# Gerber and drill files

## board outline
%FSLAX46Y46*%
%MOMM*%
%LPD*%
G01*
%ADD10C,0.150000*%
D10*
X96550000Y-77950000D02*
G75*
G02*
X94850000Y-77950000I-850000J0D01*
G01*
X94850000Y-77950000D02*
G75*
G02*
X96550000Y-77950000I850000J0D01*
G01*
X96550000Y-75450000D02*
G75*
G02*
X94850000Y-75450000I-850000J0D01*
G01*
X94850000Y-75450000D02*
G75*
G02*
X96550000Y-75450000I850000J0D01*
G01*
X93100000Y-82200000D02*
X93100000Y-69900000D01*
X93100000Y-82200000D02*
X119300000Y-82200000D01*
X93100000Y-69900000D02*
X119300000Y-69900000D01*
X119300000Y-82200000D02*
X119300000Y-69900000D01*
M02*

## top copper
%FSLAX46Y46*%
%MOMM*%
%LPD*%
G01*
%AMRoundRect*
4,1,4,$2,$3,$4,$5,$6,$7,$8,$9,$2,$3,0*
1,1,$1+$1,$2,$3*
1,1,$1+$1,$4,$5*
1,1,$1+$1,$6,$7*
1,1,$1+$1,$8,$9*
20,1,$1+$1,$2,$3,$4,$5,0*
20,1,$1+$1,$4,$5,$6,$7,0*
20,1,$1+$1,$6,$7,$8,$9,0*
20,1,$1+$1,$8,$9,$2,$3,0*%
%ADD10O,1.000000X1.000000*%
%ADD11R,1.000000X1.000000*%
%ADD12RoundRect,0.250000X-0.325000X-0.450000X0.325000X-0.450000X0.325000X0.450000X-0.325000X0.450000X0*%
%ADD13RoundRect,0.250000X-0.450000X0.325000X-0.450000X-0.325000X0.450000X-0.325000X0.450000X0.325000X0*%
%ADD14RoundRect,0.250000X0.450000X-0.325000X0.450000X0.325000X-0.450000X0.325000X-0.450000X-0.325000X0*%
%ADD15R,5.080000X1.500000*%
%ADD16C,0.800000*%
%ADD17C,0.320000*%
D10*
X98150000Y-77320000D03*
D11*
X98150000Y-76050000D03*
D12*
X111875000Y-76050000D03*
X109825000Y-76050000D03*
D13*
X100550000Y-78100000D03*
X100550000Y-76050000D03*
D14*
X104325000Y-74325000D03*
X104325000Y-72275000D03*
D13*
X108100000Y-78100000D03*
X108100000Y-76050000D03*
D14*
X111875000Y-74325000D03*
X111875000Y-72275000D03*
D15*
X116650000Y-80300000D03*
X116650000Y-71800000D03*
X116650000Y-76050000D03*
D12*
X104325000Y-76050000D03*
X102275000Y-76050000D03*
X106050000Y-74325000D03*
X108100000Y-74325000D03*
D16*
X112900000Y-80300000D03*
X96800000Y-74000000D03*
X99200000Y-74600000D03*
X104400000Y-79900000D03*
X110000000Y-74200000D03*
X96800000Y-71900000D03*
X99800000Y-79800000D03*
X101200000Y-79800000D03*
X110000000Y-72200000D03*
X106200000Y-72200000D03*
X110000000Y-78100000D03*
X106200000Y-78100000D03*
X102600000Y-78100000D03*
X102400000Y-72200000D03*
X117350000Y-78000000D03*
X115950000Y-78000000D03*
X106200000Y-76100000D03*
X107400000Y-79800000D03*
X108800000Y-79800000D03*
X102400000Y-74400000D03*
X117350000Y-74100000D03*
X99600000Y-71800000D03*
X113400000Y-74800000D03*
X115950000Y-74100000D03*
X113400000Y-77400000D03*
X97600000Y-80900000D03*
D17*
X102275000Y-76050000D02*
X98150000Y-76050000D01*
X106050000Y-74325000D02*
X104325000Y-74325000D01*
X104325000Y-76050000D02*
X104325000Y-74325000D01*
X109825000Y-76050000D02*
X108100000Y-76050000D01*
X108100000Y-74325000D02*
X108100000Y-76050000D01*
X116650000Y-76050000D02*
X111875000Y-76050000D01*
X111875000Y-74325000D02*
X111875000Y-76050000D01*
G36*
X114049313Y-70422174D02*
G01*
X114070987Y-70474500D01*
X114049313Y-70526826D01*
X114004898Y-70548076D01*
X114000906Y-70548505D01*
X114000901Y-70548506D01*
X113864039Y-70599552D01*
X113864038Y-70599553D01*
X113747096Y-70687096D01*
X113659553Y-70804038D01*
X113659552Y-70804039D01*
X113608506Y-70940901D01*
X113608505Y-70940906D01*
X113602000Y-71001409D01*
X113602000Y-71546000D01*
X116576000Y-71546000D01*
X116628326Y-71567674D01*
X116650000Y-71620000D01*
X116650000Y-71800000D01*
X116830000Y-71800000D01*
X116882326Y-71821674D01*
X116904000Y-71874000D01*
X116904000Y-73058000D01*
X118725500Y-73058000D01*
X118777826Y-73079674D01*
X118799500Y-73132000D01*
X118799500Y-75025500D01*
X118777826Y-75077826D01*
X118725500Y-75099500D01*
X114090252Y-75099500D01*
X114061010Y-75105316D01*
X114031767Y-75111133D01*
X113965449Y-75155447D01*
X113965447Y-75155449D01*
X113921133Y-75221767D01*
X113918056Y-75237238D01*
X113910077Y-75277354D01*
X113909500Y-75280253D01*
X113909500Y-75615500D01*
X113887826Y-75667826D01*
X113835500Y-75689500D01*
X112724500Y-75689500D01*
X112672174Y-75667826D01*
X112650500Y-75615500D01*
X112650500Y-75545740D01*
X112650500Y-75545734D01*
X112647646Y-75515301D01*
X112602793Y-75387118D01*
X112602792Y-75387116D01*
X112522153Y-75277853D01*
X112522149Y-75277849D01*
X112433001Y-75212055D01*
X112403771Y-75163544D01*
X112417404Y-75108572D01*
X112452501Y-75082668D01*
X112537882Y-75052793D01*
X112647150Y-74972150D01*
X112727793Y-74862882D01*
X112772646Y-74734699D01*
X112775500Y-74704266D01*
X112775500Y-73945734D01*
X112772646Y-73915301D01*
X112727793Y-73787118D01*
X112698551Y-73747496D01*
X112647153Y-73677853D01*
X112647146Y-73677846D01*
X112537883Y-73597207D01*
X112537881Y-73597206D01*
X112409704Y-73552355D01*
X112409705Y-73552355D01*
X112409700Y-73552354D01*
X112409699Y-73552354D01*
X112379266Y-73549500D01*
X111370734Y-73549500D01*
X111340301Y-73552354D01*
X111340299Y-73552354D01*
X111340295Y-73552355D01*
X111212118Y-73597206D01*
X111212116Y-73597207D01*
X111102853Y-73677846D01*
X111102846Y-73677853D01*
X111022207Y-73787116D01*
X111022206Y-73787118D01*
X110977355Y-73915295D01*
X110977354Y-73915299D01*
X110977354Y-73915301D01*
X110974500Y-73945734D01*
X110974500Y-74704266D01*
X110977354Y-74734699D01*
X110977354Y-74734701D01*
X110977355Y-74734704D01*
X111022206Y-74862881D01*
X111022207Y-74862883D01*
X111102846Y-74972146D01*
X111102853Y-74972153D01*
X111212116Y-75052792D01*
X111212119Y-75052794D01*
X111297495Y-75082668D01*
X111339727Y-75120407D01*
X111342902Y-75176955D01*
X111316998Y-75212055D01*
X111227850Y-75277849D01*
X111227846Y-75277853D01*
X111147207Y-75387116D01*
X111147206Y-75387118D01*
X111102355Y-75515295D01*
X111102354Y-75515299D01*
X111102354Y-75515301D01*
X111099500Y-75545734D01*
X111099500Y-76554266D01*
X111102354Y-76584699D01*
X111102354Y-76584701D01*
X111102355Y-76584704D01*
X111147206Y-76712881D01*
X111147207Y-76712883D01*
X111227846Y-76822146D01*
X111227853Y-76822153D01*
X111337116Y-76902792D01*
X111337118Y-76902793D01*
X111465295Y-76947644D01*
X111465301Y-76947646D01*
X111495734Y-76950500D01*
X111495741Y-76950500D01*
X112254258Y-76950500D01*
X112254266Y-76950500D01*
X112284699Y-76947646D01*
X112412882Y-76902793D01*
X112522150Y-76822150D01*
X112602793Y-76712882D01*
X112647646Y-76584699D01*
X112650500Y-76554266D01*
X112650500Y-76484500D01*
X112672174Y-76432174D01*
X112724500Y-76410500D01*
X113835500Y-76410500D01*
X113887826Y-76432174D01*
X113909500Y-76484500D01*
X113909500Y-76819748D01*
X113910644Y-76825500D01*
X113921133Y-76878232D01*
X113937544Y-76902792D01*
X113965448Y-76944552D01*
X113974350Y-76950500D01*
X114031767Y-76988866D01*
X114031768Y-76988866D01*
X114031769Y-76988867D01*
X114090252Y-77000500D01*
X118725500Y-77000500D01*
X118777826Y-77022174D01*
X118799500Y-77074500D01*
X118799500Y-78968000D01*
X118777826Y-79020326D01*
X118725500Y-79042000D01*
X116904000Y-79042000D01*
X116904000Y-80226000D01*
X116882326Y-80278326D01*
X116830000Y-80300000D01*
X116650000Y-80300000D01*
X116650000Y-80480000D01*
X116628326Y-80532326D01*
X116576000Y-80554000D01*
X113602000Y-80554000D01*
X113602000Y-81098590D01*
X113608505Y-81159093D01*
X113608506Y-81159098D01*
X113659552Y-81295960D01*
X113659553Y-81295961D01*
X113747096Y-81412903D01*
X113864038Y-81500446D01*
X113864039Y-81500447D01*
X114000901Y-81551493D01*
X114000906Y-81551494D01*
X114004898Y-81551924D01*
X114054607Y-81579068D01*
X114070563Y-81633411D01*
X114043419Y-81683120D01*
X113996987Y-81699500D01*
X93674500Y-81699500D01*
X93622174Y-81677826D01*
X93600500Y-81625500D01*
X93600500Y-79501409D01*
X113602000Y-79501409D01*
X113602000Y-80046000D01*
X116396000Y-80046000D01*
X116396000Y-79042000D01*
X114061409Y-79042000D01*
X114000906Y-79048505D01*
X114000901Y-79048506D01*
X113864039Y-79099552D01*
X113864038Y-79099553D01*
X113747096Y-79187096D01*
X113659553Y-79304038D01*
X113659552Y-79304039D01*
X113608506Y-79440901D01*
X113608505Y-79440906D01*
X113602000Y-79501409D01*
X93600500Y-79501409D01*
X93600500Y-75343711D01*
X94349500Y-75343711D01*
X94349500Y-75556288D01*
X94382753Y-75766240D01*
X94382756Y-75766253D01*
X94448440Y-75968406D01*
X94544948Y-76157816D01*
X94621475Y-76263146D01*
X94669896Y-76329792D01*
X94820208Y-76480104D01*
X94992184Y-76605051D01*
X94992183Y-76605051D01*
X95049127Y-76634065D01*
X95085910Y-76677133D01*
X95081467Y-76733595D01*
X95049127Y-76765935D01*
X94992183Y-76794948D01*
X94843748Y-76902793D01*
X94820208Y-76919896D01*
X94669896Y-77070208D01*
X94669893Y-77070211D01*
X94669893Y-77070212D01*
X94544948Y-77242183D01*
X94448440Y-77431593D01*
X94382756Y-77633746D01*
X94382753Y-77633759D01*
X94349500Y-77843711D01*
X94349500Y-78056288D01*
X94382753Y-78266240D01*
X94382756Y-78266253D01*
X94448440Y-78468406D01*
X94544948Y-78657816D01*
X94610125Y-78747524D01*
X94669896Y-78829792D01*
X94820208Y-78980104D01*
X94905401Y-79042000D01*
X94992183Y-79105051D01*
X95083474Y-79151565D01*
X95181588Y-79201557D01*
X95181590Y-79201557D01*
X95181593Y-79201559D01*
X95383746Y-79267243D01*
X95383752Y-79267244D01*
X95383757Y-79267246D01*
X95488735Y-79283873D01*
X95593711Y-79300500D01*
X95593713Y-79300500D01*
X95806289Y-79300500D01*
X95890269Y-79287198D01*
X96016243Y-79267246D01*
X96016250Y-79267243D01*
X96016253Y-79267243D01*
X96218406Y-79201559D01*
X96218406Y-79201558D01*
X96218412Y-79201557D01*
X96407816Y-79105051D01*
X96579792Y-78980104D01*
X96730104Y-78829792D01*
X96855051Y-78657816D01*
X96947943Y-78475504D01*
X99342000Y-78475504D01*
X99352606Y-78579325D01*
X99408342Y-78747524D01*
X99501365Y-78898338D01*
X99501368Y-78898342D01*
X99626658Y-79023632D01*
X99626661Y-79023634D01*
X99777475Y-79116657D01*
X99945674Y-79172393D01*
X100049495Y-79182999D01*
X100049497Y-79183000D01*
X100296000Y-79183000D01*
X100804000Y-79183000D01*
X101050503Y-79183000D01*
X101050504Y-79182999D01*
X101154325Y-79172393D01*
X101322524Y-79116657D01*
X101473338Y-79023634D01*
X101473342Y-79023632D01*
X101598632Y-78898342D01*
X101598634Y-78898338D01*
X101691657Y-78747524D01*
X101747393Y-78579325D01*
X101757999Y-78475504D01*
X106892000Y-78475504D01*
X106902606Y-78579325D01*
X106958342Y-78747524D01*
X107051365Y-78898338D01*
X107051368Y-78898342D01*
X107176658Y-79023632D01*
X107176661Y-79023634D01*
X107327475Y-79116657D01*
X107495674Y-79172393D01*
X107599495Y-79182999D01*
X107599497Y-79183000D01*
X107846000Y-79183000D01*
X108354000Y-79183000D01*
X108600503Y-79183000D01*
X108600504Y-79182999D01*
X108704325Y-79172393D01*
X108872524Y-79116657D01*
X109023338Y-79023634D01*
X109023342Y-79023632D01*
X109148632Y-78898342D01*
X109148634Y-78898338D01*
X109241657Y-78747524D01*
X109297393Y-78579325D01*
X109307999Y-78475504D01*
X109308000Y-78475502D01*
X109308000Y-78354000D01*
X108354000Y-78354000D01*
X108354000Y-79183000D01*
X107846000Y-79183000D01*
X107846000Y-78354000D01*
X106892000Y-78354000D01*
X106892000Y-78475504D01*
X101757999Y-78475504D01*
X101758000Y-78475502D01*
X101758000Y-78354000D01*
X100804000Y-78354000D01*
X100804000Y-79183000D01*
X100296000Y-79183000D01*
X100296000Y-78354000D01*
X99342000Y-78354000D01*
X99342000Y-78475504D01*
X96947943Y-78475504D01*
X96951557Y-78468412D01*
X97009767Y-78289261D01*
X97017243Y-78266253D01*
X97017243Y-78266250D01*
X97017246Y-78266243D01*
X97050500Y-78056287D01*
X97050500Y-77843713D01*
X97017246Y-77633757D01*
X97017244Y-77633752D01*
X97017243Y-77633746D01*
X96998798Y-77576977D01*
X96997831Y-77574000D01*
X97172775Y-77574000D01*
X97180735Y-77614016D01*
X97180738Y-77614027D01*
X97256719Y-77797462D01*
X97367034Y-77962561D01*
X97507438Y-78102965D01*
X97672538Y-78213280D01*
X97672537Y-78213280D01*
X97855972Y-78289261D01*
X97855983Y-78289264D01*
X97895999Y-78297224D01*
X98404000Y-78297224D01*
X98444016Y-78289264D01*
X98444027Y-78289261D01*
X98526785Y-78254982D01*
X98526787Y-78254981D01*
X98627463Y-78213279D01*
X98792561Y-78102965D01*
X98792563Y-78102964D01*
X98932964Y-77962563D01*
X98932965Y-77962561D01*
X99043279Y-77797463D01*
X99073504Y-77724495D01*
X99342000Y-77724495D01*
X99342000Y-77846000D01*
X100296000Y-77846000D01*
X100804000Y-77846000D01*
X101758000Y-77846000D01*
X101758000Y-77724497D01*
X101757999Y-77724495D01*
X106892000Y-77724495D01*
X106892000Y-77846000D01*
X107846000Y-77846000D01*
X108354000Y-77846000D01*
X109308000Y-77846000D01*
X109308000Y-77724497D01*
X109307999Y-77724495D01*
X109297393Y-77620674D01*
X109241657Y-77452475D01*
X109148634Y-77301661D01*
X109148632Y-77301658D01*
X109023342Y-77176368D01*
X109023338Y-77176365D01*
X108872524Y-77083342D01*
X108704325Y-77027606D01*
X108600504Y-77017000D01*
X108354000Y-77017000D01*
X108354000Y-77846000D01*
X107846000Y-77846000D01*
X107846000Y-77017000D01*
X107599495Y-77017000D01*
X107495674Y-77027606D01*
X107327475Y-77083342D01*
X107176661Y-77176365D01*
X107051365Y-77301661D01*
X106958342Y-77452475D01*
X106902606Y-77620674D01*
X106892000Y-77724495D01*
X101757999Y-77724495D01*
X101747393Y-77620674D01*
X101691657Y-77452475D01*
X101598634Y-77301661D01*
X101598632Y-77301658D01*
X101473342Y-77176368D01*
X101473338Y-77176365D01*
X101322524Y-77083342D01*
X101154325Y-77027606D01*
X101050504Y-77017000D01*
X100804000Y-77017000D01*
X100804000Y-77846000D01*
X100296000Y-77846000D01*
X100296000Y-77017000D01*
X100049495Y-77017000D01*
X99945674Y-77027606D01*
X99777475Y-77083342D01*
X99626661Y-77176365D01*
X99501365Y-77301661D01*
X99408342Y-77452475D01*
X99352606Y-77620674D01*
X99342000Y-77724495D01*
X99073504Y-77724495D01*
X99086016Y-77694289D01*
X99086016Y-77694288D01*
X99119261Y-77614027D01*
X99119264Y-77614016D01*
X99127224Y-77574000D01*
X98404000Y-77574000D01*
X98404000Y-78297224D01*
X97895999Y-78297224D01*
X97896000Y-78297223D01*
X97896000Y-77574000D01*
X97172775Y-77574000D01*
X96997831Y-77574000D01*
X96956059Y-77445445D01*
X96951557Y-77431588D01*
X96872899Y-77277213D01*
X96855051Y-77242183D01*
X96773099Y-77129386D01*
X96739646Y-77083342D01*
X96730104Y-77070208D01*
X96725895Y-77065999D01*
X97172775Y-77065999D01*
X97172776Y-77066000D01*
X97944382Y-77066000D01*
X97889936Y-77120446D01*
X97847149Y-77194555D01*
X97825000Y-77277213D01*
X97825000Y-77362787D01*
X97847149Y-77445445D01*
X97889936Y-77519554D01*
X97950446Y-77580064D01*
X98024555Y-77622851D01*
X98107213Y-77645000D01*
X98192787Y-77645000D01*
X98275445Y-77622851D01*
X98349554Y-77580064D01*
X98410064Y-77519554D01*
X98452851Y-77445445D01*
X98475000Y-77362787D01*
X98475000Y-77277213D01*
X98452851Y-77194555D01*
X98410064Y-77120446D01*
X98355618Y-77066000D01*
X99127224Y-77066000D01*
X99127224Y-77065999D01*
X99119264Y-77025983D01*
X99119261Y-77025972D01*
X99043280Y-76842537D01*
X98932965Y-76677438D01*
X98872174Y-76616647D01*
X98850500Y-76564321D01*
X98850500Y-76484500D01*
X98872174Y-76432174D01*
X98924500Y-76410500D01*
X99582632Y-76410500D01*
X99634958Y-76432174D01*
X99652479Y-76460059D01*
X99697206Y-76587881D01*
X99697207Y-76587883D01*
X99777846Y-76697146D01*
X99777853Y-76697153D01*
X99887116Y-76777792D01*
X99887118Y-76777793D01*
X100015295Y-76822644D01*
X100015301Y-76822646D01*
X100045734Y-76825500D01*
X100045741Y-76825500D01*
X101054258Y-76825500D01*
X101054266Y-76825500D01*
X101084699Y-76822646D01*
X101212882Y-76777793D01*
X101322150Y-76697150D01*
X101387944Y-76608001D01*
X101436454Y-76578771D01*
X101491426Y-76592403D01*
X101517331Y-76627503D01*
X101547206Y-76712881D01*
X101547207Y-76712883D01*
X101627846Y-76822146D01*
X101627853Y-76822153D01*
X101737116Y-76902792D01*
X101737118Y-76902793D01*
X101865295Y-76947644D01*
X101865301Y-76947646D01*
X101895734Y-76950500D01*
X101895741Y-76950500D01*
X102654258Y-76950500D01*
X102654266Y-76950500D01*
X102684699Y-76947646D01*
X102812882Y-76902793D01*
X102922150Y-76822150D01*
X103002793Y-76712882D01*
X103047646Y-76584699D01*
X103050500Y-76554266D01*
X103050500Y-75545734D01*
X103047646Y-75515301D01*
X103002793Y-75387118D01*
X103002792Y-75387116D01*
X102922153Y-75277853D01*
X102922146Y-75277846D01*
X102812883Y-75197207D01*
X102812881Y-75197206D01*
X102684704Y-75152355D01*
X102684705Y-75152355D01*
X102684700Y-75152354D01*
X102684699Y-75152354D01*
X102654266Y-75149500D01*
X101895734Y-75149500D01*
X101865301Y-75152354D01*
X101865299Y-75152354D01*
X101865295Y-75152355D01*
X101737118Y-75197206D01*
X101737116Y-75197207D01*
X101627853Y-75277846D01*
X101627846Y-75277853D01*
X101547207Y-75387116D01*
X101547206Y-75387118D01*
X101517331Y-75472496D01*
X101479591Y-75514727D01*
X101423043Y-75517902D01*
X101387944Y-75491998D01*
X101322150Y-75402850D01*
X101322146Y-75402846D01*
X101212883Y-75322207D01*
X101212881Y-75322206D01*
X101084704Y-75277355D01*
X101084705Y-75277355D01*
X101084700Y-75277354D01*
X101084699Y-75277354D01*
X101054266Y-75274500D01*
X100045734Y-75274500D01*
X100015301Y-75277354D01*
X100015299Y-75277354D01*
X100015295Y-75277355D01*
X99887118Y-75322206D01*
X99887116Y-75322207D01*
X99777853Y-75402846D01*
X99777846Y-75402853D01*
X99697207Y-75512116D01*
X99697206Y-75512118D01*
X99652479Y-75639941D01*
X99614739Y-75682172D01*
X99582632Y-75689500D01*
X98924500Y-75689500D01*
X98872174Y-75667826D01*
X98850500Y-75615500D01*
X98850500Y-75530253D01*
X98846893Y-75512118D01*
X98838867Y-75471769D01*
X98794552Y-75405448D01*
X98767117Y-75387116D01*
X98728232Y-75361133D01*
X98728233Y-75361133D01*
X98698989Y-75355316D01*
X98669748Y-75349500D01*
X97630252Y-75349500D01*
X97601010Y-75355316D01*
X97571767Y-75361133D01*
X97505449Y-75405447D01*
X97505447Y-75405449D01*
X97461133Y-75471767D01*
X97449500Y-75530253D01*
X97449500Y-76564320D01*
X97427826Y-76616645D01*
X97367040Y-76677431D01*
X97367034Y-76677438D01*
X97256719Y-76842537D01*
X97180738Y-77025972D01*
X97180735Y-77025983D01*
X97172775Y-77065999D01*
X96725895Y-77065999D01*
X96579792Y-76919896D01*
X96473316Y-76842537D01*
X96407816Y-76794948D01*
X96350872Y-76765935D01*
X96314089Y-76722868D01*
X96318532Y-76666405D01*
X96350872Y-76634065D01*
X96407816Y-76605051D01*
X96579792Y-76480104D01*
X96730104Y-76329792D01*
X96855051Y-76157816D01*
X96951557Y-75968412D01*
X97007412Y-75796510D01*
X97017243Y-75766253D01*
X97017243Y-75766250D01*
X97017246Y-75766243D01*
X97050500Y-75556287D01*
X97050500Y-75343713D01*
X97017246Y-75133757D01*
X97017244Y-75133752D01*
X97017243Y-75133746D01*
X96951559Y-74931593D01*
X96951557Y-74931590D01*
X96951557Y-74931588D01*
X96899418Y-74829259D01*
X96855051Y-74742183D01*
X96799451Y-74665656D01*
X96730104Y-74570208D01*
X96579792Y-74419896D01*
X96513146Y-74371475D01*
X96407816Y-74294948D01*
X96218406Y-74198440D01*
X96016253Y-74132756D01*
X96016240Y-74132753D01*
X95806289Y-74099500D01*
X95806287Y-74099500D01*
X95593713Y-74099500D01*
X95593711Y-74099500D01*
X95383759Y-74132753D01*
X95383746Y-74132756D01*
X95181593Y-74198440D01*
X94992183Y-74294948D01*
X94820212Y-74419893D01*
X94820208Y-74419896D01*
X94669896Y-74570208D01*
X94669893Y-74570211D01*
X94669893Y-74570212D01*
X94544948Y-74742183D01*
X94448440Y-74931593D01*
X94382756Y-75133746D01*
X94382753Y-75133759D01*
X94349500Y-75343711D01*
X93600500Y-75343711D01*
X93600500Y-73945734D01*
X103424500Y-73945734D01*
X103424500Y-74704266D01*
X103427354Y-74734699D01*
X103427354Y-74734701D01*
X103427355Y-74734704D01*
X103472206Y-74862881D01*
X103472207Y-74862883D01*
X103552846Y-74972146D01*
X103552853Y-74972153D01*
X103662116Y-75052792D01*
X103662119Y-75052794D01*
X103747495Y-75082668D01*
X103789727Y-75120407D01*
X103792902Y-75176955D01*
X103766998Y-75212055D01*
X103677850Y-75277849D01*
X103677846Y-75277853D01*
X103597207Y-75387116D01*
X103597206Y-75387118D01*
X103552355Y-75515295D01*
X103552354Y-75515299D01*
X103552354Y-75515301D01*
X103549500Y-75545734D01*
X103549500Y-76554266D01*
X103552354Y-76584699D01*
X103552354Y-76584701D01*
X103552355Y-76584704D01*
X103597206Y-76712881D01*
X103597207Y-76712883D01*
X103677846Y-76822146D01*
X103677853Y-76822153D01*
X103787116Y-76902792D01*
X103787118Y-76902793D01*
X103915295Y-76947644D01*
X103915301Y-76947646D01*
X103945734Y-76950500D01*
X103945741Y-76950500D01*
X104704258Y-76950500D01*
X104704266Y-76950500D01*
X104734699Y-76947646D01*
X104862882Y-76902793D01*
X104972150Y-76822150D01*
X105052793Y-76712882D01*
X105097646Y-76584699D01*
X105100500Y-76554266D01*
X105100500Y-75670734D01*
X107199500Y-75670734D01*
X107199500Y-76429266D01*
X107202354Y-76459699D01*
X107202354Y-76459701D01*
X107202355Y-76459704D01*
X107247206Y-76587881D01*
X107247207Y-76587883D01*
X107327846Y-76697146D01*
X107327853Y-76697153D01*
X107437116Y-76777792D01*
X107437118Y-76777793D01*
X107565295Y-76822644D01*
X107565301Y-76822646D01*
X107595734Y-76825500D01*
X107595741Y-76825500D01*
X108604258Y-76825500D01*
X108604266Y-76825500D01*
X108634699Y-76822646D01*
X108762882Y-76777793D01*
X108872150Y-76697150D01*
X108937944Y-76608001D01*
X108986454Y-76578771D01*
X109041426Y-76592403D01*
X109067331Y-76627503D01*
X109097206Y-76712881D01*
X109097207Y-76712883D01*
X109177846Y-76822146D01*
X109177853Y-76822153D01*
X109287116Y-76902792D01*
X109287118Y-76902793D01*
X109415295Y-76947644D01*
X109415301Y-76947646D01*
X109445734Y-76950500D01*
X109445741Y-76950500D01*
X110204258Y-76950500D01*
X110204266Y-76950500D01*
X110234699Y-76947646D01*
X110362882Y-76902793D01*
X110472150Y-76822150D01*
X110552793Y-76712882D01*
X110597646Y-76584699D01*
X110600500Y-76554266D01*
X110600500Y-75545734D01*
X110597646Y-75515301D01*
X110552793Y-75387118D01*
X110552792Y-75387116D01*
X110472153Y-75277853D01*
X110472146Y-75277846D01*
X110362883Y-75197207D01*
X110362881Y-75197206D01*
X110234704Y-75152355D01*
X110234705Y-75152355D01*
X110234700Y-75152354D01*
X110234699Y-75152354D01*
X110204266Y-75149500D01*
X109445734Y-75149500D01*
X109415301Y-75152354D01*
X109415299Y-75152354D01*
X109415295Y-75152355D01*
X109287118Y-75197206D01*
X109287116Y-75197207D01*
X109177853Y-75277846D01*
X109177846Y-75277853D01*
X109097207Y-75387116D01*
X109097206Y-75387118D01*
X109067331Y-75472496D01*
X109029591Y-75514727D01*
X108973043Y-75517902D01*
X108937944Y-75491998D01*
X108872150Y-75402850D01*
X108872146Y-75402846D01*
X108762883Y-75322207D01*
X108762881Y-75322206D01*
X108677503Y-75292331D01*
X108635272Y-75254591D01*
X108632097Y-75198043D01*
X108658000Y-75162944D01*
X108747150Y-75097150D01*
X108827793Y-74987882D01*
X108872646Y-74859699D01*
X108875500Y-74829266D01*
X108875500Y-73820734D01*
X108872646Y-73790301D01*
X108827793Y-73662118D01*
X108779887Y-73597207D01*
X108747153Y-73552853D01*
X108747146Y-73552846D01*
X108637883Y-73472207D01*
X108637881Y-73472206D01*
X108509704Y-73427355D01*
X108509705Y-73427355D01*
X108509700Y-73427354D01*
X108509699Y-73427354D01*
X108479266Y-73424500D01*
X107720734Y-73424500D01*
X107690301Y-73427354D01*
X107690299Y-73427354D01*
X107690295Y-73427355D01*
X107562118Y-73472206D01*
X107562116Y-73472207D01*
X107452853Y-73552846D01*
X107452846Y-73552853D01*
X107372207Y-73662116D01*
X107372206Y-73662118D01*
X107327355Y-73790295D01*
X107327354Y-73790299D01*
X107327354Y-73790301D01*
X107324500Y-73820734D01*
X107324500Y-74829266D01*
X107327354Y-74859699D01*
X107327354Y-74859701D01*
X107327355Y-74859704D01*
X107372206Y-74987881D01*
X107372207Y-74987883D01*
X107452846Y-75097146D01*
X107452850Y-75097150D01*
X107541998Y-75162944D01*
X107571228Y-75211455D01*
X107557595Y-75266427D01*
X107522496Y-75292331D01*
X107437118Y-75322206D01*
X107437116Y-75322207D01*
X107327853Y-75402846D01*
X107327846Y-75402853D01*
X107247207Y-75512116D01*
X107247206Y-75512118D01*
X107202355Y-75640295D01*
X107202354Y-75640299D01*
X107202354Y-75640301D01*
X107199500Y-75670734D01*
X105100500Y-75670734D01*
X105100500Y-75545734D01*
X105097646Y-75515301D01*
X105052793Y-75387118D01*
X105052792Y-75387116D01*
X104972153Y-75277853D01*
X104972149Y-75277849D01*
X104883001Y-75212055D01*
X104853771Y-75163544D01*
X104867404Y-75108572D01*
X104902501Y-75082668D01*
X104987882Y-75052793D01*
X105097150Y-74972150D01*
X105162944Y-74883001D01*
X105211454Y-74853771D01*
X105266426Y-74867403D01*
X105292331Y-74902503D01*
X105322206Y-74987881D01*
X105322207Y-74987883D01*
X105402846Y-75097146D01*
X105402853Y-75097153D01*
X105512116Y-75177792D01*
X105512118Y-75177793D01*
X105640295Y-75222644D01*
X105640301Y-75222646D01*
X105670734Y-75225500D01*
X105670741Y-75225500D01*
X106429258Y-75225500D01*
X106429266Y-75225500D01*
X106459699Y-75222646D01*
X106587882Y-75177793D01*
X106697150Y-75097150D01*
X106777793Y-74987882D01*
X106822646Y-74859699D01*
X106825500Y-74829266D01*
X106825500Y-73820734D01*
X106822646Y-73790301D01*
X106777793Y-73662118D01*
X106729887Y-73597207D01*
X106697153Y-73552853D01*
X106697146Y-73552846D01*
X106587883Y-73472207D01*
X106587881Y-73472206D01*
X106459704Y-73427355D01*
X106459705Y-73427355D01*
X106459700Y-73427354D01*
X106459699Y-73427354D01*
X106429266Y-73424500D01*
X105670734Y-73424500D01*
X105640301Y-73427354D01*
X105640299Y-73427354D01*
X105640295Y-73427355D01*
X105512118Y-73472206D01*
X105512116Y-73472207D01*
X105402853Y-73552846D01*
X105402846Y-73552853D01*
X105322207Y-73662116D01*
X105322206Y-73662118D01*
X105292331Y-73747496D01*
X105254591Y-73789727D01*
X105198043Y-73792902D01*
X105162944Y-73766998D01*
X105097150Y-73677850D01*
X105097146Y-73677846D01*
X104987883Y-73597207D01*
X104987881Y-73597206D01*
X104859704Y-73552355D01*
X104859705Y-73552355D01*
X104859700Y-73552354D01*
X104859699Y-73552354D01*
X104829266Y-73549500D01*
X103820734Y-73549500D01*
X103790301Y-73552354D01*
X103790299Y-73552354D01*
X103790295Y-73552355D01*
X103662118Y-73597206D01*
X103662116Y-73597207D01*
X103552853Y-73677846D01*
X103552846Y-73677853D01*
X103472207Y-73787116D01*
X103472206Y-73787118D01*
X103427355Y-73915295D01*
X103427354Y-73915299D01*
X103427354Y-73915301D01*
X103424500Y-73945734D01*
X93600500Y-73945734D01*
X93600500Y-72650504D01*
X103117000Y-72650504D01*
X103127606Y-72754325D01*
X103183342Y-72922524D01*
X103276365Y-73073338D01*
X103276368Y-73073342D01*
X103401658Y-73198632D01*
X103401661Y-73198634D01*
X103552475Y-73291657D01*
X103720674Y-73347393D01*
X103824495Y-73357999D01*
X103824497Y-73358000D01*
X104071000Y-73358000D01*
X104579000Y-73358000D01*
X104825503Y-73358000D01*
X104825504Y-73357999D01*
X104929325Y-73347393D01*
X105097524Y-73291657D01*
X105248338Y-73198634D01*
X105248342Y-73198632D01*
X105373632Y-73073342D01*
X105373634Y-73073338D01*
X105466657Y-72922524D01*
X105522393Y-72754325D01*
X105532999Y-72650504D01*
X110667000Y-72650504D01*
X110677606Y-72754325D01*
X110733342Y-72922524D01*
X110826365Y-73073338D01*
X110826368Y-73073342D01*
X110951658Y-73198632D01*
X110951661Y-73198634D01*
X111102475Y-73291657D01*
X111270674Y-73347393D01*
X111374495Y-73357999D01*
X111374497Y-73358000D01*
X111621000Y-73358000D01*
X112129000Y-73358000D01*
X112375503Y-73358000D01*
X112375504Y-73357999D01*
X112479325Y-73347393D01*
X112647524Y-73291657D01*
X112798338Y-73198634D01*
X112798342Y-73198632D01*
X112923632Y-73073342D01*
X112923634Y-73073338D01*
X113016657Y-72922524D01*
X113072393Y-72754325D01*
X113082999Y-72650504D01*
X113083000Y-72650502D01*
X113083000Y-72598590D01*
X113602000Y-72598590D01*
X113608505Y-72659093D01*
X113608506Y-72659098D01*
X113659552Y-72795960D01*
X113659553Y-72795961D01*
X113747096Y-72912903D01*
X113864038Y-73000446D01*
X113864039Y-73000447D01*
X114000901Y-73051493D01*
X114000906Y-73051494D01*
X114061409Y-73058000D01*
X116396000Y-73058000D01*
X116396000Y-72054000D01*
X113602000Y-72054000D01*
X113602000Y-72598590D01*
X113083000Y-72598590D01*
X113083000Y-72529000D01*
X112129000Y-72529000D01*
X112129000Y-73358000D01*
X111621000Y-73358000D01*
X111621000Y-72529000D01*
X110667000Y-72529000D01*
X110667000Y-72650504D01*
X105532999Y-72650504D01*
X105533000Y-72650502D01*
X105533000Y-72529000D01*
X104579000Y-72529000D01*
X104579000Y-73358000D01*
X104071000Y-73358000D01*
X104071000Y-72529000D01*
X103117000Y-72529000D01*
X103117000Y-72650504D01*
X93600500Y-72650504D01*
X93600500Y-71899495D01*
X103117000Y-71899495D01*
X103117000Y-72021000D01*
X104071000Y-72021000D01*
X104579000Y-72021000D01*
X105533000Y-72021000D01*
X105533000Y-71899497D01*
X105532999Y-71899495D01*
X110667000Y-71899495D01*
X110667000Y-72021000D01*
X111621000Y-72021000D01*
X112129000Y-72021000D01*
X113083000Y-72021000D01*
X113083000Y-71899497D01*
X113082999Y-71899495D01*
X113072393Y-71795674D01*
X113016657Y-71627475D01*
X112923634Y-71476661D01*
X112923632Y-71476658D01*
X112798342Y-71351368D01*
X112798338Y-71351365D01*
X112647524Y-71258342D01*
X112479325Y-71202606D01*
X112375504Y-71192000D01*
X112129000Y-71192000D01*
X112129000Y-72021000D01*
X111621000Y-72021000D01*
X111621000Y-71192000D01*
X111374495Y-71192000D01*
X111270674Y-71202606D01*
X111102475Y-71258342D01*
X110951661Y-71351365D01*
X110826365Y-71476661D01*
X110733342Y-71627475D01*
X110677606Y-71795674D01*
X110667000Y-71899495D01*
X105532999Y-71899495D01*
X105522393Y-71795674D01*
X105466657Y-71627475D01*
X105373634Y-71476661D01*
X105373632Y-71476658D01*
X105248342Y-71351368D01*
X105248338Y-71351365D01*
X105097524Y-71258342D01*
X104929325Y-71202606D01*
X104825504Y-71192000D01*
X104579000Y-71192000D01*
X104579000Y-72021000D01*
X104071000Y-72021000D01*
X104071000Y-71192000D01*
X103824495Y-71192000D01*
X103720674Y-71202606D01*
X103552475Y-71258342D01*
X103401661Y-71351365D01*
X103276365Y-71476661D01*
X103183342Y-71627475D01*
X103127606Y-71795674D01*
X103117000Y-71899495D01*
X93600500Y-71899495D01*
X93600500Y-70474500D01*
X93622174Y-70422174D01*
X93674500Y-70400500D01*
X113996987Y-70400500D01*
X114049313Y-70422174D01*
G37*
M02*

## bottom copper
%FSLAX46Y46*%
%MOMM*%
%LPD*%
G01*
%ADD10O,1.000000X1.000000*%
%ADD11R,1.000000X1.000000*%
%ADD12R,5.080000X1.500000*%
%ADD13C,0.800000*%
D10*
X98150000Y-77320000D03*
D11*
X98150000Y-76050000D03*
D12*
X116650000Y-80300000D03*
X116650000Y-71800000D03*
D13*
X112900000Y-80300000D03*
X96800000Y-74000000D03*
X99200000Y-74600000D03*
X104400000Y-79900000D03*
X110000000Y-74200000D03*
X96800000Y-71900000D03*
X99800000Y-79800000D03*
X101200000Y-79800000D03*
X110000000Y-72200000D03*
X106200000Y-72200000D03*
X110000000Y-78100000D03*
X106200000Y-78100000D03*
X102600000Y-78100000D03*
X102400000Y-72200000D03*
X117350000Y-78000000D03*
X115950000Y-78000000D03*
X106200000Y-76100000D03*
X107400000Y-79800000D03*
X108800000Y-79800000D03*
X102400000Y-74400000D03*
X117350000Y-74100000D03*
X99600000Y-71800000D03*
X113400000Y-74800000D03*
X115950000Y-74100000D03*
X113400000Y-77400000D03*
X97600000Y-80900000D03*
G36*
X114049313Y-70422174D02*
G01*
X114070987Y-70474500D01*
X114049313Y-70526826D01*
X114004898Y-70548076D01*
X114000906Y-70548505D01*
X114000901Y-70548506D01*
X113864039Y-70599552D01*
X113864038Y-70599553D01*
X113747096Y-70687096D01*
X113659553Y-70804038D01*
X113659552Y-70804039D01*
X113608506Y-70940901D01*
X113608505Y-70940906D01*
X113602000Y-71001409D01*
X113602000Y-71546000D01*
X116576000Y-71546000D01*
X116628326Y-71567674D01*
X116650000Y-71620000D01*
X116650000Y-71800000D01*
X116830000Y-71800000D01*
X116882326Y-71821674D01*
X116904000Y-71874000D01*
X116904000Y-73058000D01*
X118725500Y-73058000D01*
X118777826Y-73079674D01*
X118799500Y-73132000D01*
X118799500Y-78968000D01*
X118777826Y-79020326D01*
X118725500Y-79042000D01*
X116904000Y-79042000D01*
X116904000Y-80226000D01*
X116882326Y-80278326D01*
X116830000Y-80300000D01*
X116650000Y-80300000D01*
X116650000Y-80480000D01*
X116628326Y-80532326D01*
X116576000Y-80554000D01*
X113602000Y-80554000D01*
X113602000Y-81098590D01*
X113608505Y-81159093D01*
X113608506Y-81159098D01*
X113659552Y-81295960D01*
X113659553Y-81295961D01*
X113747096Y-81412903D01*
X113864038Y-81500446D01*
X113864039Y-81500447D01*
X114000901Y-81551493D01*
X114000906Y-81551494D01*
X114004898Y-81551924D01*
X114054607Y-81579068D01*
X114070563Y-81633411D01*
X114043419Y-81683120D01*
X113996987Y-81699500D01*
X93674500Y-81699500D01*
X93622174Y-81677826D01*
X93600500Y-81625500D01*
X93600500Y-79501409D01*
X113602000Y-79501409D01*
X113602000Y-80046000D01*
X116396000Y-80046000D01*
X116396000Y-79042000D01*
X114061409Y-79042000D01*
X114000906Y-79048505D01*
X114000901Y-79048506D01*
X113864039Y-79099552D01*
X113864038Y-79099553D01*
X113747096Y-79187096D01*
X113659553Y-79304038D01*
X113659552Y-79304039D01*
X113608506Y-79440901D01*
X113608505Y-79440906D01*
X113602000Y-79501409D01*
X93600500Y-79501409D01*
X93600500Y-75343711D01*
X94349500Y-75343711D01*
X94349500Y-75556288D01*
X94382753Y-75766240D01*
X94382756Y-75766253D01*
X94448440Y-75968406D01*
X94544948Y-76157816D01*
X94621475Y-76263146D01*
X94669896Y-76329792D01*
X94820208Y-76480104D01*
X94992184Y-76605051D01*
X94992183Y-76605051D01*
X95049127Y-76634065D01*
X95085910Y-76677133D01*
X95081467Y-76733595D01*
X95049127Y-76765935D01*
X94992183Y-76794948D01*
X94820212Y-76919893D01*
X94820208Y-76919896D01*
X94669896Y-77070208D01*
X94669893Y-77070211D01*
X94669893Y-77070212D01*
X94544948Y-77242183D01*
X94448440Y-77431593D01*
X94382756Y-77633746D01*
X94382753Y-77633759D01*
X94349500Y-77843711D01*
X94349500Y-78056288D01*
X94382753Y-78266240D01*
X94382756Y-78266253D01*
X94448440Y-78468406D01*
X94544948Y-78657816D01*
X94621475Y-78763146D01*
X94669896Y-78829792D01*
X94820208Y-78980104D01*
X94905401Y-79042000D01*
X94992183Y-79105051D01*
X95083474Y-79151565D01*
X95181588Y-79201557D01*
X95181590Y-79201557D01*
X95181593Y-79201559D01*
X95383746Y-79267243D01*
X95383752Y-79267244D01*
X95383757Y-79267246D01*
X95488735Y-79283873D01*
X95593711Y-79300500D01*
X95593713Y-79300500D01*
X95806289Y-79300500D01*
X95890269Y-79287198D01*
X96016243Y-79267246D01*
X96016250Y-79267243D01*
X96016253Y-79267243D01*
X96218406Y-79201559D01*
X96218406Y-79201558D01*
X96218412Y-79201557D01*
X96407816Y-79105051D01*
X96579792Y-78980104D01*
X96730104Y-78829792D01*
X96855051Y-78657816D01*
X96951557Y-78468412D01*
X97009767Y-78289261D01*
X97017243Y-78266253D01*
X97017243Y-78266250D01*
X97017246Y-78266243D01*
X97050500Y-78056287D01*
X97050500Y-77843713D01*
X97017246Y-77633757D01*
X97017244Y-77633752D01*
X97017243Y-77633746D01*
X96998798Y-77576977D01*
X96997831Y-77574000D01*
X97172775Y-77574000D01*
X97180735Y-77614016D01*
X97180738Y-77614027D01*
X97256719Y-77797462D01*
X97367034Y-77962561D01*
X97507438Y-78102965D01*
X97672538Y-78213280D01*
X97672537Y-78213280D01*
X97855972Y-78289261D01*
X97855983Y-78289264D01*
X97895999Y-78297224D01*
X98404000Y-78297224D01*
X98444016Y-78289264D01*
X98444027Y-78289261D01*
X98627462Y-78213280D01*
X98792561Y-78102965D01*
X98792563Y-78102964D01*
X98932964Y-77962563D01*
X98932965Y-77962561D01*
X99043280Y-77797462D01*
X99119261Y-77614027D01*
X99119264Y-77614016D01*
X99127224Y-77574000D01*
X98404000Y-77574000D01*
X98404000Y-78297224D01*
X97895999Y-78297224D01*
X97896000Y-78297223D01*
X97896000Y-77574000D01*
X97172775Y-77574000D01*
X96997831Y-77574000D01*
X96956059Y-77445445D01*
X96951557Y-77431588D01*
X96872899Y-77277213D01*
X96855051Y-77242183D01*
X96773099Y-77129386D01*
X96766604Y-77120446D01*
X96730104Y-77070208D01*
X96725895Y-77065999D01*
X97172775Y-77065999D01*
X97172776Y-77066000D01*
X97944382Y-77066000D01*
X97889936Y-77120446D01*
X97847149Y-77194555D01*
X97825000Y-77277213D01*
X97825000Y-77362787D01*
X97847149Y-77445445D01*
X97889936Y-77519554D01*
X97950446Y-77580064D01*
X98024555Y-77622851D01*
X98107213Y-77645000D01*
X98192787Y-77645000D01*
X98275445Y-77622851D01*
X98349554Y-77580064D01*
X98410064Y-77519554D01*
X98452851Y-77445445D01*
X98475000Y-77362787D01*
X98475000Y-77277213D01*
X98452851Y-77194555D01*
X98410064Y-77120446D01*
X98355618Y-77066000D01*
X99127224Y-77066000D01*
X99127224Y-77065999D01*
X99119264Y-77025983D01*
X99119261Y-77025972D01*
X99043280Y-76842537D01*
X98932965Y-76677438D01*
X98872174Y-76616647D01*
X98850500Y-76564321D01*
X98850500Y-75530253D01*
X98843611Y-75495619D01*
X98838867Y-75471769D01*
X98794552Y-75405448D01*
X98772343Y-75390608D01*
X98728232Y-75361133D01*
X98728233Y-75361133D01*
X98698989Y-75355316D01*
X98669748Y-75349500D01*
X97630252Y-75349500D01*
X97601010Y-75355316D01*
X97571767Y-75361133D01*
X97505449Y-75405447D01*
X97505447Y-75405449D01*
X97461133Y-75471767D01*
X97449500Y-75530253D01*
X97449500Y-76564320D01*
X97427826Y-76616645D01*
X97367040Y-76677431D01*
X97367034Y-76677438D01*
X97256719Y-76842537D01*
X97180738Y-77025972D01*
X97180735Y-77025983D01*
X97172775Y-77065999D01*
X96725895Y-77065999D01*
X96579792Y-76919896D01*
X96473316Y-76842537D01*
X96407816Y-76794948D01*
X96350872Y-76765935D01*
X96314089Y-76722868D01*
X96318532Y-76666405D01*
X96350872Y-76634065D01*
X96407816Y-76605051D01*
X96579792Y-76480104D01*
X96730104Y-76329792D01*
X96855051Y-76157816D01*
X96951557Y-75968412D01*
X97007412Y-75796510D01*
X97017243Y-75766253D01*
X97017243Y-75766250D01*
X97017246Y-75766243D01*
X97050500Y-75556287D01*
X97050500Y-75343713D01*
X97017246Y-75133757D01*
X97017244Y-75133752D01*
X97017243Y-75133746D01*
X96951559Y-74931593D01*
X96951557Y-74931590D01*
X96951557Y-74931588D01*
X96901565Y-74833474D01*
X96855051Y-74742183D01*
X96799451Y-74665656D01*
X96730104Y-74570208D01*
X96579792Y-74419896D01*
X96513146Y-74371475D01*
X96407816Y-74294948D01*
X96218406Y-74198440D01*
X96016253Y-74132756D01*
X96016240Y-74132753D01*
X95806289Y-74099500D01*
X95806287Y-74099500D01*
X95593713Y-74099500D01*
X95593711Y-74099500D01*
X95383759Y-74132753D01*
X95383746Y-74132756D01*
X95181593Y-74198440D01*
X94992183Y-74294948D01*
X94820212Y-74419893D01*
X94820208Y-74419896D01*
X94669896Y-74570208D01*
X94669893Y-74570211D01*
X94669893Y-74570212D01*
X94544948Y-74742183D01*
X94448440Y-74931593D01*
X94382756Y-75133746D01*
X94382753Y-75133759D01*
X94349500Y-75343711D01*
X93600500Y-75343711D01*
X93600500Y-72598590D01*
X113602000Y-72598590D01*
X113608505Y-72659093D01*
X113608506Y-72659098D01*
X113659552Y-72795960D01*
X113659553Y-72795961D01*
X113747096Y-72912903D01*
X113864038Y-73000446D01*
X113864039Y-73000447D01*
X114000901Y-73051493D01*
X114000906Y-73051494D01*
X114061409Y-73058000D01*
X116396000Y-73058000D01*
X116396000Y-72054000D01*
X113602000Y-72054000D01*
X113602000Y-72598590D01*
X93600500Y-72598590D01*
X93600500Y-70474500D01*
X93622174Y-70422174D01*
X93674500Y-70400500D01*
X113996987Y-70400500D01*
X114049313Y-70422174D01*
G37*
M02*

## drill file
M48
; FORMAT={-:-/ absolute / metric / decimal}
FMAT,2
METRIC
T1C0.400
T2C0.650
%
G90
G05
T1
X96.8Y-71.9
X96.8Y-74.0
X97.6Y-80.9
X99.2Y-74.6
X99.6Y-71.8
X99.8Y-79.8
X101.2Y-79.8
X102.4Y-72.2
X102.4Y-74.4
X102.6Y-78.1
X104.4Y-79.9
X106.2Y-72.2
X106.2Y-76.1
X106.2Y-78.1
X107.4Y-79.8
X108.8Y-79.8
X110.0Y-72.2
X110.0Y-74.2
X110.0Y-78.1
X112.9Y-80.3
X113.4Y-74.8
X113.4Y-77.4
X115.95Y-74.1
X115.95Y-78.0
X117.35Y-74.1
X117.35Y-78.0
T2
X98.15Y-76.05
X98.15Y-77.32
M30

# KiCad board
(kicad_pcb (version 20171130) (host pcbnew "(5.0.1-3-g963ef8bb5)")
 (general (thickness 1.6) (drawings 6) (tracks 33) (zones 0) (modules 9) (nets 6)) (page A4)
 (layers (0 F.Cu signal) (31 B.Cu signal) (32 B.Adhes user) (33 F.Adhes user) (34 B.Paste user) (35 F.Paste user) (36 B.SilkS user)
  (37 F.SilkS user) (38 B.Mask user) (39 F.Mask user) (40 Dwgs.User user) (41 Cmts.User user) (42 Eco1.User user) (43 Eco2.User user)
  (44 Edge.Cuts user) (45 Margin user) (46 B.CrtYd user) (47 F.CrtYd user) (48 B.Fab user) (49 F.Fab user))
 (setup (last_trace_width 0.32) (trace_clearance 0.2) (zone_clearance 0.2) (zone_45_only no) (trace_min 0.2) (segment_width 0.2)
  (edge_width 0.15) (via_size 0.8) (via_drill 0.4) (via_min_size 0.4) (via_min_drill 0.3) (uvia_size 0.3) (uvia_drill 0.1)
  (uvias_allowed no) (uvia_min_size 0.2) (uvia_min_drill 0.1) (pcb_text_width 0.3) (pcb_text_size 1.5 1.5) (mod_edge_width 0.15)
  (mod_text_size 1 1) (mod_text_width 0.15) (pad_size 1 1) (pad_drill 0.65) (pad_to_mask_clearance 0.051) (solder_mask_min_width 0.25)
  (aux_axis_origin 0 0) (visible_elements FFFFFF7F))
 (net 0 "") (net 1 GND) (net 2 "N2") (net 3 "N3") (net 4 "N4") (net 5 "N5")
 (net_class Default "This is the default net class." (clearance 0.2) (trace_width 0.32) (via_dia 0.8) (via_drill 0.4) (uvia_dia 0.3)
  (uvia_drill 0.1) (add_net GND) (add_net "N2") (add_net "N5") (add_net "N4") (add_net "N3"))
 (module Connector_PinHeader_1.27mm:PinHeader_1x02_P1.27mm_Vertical (layer F.Cu) (at 98.15 76.05)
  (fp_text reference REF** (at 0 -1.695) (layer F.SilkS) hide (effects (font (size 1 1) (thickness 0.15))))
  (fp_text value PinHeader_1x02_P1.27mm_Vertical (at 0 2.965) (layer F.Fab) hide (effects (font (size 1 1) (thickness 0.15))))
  (pad 2 thru_hole oval (at 0 1.27) (size 1 1) (drill 0.65) (layers *.Cu *.Mask) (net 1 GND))
  (pad 1 thru_hole rect (at 0 0) (size 1 1) (drill 0.65) (layers *.Cu *.Mask) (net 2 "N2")))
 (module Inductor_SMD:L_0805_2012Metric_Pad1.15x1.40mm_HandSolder (layer F.Cu) (at 110.85 76.05)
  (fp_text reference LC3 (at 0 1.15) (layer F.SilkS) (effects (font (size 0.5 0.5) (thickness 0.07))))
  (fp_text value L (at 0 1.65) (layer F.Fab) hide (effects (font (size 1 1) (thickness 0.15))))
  (pad 2 smd roundrect (at 1.025 0) (size 1.15 1.4) (layers F.Cu F.Paste F.Mask) (roundrect_rratio 0.217391) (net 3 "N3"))
  (pad 1 smd roundrect (at -1.025 0) (size 1.15 1.4) (layers F.Cu F.Paste F.Mask) (roundrect_rratio 0.217391) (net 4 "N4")))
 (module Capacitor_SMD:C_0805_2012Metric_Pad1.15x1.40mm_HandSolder (layer F.Cu) (at 100.55 77.075 270)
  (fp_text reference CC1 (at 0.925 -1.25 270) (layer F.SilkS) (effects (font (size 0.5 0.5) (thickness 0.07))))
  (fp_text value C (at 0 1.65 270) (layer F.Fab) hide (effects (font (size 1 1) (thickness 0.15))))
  (pad 2 smd roundrect (at 1.025 0 270) (size 1.15 1.4) (layers F.Cu F.Paste F.Mask) (roundrect_rratio 0.217391) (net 1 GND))
  (pad 1 smd roundrect (at -1.025 0 270) (size 1.15 1.4) (layers F.Cu F.Paste F.Mask) (roundrect_rratio 0.217391) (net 2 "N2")))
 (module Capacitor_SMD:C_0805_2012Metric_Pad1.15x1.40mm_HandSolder (layer F.Cu) (at 104.325 73.3 90)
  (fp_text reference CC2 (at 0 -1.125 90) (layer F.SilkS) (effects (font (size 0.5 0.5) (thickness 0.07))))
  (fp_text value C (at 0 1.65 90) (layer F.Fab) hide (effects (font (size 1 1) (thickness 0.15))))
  (pad 1 smd roundrect (at -1.025 0 90) (size 1.15 1.4) (layers F.Cu F.Paste F.Mask) (roundrect_rratio 0.217391) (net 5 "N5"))
  (pad 2 smd roundrect (at 1.025 0 90) (size 1.15 1.4) (layers F.Cu F.Paste F.Mask) (roundrect_rratio 0.217391) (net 1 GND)))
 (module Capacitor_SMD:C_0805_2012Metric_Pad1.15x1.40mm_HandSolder (layer F.Cu) (at 108.1 77.075 270)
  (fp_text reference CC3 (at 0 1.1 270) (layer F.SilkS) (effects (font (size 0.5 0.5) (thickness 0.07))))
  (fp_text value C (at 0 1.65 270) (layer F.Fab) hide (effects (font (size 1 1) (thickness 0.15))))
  (pad 2 smd roundrect (at 1.025 0 270) (size 1.15 1.4) (layers F.Cu F.Paste F.Mask) (roundrect_rratio 0.217391) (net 1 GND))
  (pad 1 smd roundrect (at -1.025 0 270) (size 1.15 1.4) (layers F.Cu F.Paste F.Mask) (roundrect_rratio 0.217391) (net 4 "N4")))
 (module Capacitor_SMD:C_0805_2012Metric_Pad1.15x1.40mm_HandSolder (layer F.Cu) (at 111.875 73.3 90)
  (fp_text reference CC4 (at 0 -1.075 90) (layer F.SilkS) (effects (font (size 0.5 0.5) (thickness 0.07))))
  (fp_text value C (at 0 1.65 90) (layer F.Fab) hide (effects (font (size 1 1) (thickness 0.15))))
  (pad 1 smd roundrect (at -1.025 0 90) (size 1.15 1.4) (layers F.Cu F.Paste F.Mask) (roundrect_rratio 0.217391) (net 3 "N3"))
  (pad 2 smd roundrect (at 1.025 0 90) (size 1.15 1.4) (layers F.Cu F.Paste F.Mask) (roundrect_rratio 0.217391) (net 1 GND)))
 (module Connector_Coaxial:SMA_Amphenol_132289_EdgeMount (layer F.Cu) (at 116.65 76.05)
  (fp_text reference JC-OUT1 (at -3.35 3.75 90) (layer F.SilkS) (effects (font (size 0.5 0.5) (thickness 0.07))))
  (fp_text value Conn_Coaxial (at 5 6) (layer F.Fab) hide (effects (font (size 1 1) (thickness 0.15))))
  (pad 2 smd rect (at 0 4.25 90) (size 1.5 5.08) (layers B.Cu B.Paste B.Mask) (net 1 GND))
  (pad 2 smd rect (at 0 -4.25 90) (size 1.5 5.08) (layers B.Cu B.Paste B.Mask) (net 1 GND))
  (pad 2 smd rect (at 0 4.25 90) (size 1.5 5.08) (layers F.Cu F.Paste F.Mask) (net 1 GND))
  (pad 2 smd rect (at 0 -4.25 90) (size 1.5 5.08) (layers F.Cu F.Paste F.Mask) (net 1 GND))
  (pad 1 smd rect (at 0 0 90) (size 1.5 5.08) (layers F.Cu F.Paste F.Mask) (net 3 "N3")))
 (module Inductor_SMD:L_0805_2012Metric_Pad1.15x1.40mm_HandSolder (layer F.Cu) (at 103.3 76.05)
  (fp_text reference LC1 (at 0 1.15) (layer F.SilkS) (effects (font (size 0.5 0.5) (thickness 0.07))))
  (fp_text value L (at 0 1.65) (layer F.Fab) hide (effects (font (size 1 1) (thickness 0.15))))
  (pad 2 smd roundrect (at 1.025 0) (size 1.15 1.4) (layers F.Cu F.Paste F.Mask) (roundrect_rratio 0.217391) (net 5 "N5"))
  (pad 1 smd roundrect (at -1.025 0) (size 1.15 1.4) (layers F.Cu F.Paste F.Mask) (roundrect_rratio 0.217391) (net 2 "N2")))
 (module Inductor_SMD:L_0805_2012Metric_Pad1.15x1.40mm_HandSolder (layer F.Cu) (at 107.075 74.325)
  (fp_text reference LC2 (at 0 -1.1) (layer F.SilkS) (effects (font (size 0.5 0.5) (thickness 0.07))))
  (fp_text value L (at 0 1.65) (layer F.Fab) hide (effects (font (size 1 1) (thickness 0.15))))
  (pad 1 smd roundrect (at -1.025 0) (size 1.15 1.4) (layers F.Cu F.Paste F.Mask) (roundrect_rratio 0.217391) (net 5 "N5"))
  (pad 2 smd roundrect (at 1.025 0) (size 1.15 1.4) (layers F.Cu F.Paste F.Mask) (roundrect_rratio 0.217391) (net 4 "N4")))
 (gr_circle (center 95.7 77.95) (end 96.55 77.95) (layer Edge.Cuts) (width 0.15))
 (gr_circle (center 95.7 75.45) (end 96.55 75.45) (layer Edge.Cuts) (width 0.15))
 (gr_line (start 93.1 82.2) (end 93.1 69.9) (layer Edge.Cuts) (width 0.15))
 (gr_line (start 93.1 82.2) (end 119.3 82.2) (layer Edge.Cuts) (width 0.15))
 (gr_line (start 93.1 69.9) (end 119.3 69.9) (layer Edge.Cuts) (width 0.15))
 (gr_line (start 119.3 82.2) (end 119.3 69.9) (layer Edge.Cuts) (width 0.15))
 (via (at 112.9 80.3) (size 0.8) (drill 0.4) (layers F.Cu B.Cu) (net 1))
 (via (at 96.8 74) (size 0.8) (drill 0.4) (layers F.Cu B.Cu) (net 1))
 (via (at 99.2 74.6) (size 0.8) (drill 0.4) (layers F.Cu B.Cu) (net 1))
 (via (at 104.4 79.9) (size 0.8) (drill 0.4) (layers F.Cu B.Cu) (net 1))
 (via (at 110 74.2) (size 0.8) (drill 0.4) (layers F.Cu B.Cu) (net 1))
 (via (at 96.8 71.9) (size 0.8) (drill 0.4) (layers F.Cu B.Cu) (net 1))
 (via (at 99.8 79.8) (size 0.8) (drill 0.4) (layers F.Cu B.Cu) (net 1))
 (via (at 101.2 79.8) (size 0.8) (drill 0.4) (layers F.Cu B.Cu) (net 1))
 (via (at 110 72.2) (size 0.8) (drill 0.4) (layers F.Cu B.Cu) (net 1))
 (via (at 106.2 72.2) (size 0.8) (drill 0.4) (layers F.Cu B.Cu) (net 1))
 (via (at 110 78.1) (size 0.8) (drill 0.4) (layers F.Cu B.Cu) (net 1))
 (via (at 106.2 78.1) (size 0.8) (drill 0.4) (layers F.Cu B.Cu) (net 1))
 (via (at 102.6 78.1) (size 0.8) (drill 0.4) (layers F.Cu B.Cu) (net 1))
 (via (at 102.4 72.2) (size 0.8) (drill 0.4) (layers F.Cu B.Cu) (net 1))
 (via (at 117.35 78) (size 0.8) (drill 0.4) (layers F.Cu B.Cu) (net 1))
 (via (at 115.95 78) (size 0.8) (drill 0.4) (layers F.Cu B.Cu) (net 1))
 (via (at 106.2 76.1) (size 0.8) (drill 0.4) (layers F.Cu B.Cu) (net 1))
 (via (at 107.4 79.8) (size 0.8) (drill 0.4) (layers F.Cu B.Cu) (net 1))
 (via (at 108.8 79.8) (size 0.8) (drill 0.4) (layers F.Cu B.Cu) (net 1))
 (via (at 102.4 74.4) (size 0.8) (drill 0.4) (layers F.Cu B.Cu) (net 1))
 (via (at 117.35 74.1) (size 0.8) (drill 0.4) (layers F.Cu B.Cu) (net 1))
 (via (at 99.6 71.8) (size 0.8) (drill 0.4) (layers F.Cu B.Cu) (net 1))
 (via (at 113.4 74.8) (size 0.8) (drill 0.4) (layers F.Cu B.Cu) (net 1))
 (via (at 115.95 74.1) (size 0.8) (drill 0.4) (layers F.Cu B.Cu) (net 1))
 (via (at 113.4 77.4) (size 0.8) (drill 0.4) (layers F.Cu B.Cu) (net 1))
 (via (at 97.6 80.9) (size 0.8) (drill 0.4) (layers F.Cu B.Cu) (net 1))
 (segment (start 102.275 76.05) (end 98.15 76.05) (width 0.32) (layer F.Cu) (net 2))
 (segment (start 106.05 74.325) (end 104.325 74.325) (width 0.32) (layer F.Cu) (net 5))
 (segment (start 104.325 76.05) (end 104.325 74.325) (width 0.32) (layer F.Cu) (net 5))
 (segment (start 109.825 76.05) (end 108.1 76.05) (width 0.32) (layer F.Cu) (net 4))
 (segment (start 108.1 74.325) (end 108.1 76.05) (width 0.32) (layer F.Cu) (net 4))
 (segment (start 116.65 76.05) (end 111.875 76.05) (width 0.32) (layer F.Cu) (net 3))
 (segment (start 111.875 74.325) (end 111.875 76.05) (width 0.32) (layer F.Cu) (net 3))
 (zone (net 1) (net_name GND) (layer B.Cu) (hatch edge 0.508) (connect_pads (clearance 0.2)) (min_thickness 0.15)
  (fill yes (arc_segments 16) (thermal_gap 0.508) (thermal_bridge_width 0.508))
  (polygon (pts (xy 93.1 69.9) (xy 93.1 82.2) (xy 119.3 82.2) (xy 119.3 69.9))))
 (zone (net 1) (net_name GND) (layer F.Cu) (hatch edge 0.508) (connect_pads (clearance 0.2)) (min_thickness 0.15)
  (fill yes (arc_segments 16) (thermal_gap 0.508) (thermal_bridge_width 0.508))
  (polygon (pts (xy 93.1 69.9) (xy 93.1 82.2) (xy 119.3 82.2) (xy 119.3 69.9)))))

